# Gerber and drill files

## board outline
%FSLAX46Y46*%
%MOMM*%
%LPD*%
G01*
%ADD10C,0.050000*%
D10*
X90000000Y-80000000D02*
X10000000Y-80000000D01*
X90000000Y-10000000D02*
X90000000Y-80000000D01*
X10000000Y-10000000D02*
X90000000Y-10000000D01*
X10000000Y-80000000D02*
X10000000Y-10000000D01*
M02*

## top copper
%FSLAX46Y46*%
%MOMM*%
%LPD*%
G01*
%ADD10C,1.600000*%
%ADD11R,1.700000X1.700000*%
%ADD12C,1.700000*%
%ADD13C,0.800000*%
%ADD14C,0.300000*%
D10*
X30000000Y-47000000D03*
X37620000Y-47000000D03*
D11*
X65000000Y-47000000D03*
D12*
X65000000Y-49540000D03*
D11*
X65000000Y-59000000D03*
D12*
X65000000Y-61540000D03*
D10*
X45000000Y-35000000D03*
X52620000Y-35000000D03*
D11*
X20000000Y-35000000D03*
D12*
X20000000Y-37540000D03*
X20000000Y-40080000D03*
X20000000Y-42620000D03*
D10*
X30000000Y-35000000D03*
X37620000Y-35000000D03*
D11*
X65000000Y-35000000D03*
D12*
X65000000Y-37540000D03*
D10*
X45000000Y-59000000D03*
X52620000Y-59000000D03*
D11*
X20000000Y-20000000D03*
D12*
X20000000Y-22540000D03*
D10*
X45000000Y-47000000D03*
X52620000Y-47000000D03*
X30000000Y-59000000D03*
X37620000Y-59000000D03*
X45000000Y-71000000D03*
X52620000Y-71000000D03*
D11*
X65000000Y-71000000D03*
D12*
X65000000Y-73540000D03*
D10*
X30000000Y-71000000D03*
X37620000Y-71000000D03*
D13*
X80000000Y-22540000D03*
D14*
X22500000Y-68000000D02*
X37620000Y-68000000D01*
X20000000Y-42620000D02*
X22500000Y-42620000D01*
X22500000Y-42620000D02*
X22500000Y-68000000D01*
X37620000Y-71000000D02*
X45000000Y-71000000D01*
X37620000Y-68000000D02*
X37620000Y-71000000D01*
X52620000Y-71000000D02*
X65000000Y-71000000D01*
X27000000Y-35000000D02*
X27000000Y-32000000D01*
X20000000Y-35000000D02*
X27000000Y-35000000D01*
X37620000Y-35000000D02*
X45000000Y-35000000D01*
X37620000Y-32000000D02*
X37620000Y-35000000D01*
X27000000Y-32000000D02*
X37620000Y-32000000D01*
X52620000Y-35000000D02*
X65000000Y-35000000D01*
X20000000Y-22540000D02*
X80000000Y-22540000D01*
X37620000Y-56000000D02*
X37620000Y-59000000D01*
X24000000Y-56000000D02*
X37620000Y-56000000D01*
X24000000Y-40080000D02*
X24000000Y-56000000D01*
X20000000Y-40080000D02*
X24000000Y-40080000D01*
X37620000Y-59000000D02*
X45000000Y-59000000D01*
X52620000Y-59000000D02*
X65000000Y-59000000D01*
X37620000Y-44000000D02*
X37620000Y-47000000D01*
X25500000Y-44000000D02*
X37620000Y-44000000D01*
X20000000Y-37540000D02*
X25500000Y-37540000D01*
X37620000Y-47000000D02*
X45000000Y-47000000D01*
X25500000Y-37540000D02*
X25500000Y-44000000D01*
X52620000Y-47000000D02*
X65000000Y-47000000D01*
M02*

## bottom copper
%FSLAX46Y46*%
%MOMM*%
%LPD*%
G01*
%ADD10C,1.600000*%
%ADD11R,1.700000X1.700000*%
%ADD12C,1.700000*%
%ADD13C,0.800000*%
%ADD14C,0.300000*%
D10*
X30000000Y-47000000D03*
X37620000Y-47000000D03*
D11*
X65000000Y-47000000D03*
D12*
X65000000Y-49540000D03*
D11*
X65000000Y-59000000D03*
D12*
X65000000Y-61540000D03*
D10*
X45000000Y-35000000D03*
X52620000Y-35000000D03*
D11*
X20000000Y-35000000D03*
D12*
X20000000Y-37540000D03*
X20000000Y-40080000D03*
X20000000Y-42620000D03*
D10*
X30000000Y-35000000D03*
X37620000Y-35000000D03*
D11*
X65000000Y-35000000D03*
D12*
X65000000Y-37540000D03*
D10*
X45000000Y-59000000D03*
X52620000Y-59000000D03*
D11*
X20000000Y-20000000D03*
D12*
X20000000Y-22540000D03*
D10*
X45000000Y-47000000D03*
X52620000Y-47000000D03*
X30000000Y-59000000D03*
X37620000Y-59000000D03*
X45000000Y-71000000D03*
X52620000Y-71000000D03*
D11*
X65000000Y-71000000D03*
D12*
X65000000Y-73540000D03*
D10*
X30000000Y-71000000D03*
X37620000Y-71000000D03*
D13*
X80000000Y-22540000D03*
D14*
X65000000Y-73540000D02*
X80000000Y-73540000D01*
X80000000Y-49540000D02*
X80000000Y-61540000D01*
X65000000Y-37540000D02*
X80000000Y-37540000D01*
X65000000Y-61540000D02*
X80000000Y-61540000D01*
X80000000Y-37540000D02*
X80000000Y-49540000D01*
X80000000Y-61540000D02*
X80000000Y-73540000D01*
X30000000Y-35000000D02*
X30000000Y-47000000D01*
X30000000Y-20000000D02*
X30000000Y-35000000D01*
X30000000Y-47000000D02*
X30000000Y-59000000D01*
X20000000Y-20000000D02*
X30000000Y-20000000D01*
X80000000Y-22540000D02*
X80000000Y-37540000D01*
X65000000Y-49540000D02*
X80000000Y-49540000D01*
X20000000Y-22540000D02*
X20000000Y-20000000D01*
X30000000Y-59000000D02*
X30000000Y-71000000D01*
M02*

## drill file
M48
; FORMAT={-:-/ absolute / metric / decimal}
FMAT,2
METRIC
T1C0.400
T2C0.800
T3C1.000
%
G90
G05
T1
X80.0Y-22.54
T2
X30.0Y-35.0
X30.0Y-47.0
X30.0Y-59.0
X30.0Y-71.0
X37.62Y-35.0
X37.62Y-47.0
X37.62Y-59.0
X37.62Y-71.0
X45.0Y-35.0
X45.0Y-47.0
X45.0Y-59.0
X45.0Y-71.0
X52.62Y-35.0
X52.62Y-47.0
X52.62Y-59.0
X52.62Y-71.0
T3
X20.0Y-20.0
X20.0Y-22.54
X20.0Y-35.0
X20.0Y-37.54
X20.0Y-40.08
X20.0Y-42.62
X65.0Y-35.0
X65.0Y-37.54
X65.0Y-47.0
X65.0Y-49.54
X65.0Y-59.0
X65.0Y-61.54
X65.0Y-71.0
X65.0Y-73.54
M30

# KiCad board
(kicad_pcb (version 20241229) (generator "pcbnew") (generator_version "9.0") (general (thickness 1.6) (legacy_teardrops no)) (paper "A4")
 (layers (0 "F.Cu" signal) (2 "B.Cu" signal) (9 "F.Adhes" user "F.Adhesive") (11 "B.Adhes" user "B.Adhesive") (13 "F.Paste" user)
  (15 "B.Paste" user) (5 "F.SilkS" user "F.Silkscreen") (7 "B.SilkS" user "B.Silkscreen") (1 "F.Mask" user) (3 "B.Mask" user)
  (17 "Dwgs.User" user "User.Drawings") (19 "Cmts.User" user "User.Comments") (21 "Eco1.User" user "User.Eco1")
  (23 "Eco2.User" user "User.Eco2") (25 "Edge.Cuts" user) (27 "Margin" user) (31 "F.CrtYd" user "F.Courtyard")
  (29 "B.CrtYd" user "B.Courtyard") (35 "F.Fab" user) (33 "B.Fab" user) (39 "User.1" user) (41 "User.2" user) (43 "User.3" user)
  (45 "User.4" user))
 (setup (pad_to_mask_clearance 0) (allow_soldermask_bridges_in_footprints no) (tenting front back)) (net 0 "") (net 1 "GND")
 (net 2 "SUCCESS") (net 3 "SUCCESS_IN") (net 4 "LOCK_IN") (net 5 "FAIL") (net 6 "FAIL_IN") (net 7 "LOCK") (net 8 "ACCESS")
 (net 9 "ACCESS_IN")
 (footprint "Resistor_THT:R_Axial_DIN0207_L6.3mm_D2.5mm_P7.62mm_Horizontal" (layer "F.Cu") (at 30 47)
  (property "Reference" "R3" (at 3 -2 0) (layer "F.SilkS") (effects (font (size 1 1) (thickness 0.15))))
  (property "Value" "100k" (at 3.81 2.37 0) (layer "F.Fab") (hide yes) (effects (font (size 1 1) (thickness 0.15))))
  (pad "1" thru_hole circle (at 0 0) (size 1.6 1.6) (drill 0.8) (layers "*.Cu" "*.Mask") (remove_unused_layers no) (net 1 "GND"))
  (pad "2" thru_hole circle (at 7.62 0) (size 1.6 1.6) (drill 0.8) (layers "*.Cu" "*.Mask") (remove_unused_layers no) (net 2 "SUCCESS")))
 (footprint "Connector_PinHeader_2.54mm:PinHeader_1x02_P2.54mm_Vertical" (layer "F.Cu") (at 65 47)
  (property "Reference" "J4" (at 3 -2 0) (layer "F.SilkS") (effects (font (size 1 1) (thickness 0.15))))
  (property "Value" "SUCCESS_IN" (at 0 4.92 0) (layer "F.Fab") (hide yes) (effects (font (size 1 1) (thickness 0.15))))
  (pad "1" thru_hole rect (at 0 0) (size 1.7 1.7) (drill 1) (layers "*.Cu" "*.Mask") (remove_unused_layers no) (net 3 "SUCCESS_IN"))
  (pad "2" thru_hole circle (at 0 2.54) (size 1.7 1.7) (drill 1) (layers "*.Cu" "*.Mask") (remove_unused_layers no) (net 1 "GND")))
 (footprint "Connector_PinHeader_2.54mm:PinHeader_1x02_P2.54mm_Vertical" (layer "F.Cu") (at 65 59)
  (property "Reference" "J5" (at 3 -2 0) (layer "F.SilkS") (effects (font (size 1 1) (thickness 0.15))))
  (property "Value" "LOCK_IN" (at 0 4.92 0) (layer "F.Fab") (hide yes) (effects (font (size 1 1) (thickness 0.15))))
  (pad "1" thru_hole rect (at 0 0) (size 1.7 1.7) (drill 1) (layers "*.Cu" "*.Mask") (remove_unused_layers no) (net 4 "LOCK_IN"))
  (pad "2" thru_hole circle (at 0 2.54) (size 1.7 1.7) (drill 1) (layers "*.Cu" "*.Mask") (remove_unused_layers no) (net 1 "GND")))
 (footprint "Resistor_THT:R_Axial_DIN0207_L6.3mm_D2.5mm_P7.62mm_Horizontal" (layer "F.Cu") (at 45 35)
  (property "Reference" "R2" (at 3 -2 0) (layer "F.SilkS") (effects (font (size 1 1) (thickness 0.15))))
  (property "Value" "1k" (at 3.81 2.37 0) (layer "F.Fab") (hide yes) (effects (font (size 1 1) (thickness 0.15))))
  (pad "1" thru_hole circle (at 0 0) (size 1.6 1.6) (drill 0.8) (layers "*.Cu" "*.Mask") (remove_unused_layers no) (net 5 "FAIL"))
  (pad "2" thru_hole circle (at 7.62 0) (size 1.6 1.6) (drill 0.8) (layers "*.Cu" "*.Mask") (remove_unused_layers no) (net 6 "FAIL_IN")))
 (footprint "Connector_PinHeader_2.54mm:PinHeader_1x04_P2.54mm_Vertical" (layer "F.Cu") (at 20 35)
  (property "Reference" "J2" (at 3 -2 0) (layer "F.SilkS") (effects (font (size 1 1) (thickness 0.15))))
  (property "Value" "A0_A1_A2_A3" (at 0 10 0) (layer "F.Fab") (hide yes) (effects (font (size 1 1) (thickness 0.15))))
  (pad "1" thru_hole rect (at 0 0) (size 1.7 1.7) (drill 1) (layers "*.Cu" "*.Mask") (remove_unused_layers no) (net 5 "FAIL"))
  (pad "2" thru_hole circle (at 0 2.54) (size 1.7 1.7) (drill 1) (layers "*.Cu" "*.Mask") (remove_unused_layers no) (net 2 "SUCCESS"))
  (pad "3" thru_hole circle (at 0 5.08) (size 1.7 1.7) (drill 1) (layers "*.Cu" "*.Mask") (remove_unused_layers no) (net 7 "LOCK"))
  (pad "4" thru_hole circle (at 0 7.62) (size 1.7 1.7) (drill 1) (layers "*.Cu" "*.Mask") (remove_unused_layers no) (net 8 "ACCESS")))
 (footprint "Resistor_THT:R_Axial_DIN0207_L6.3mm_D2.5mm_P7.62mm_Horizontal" (layer "F.Cu") (at 30 35)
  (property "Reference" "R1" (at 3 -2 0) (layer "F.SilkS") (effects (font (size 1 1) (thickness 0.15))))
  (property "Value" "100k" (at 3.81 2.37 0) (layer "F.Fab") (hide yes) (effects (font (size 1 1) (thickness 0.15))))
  (pad "1" thru_hole circle (at 0 0) (size 1.6 1.6) (drill 0.8) (layers "*.Cu" "*.Mask") (remove_unused_layers no) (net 1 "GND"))
  (pad "2" thru_hole circle (at 7.62 0) (size 1.6 1.6) (drill 0.8) (layers "*.Cu" "*.Mask") (remove_unused_layers no) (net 5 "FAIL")))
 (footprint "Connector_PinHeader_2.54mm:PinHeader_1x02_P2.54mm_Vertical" (layer "F.Cu") (at 65 35)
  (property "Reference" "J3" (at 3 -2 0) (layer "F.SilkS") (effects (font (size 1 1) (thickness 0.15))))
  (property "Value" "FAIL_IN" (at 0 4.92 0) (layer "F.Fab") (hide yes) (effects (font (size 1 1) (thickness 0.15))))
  (pad "1" thru_hole rect (at 0 0) (size 1.7 1.7) (drill 1) (layers "*.Cu" "*.Mask") (remove_unused_layers no) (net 6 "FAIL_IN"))
  (pad "2" thru_hole circle (at 0 2.54) (size 1.7 1.7) (drill 1) (layers "*.Cu" "*.Mask") (remove_unused_layers no) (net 1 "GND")))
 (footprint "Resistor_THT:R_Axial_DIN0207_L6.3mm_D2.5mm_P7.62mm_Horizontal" (layer "F.Cu") (at 45 59)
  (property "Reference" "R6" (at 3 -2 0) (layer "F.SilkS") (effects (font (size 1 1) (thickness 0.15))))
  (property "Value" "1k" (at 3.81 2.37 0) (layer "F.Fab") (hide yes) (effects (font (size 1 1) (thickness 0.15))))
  (pad "1" thru_hole circle (at 0 0) (size 1.6 1.6) (drill 0.8) (layers "*.Cu" "*.Mask") (remove_unused_layers no) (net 7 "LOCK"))
  (pad "2" thru_hole circle (at 7.62 0) (size 1.6 1.6) (drill 0.8) (layers "*.Cu" "*.Mask") (remove_unused_layers no) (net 4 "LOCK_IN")))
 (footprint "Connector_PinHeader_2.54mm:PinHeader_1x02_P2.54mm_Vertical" (layer "F.Cu") (at 20 20)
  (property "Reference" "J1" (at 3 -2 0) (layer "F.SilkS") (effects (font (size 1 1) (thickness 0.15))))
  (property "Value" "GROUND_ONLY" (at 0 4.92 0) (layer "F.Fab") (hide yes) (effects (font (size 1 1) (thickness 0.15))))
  (pad "1" thru_hole rect (at 0 0) (size 1.7 1.7) (drill 1) (layers "*.Cu" "*.Mask") (remove_unused_layers no) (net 1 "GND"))
  (pad "2" thru_hole circle (at 0 2.54) (size 1.7 1.7) (drill 1) (layers "*.Cu" "*.Mask") (remove_unused_layers no) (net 1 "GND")))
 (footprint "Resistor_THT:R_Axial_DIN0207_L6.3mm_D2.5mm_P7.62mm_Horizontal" (layer "F.Cu") (at 45 47)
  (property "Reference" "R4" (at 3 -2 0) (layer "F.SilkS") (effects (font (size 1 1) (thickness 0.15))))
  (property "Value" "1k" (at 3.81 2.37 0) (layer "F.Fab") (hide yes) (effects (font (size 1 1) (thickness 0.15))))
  (pad "1" thru_hole circle (at 0 0) (size 1.6 1.6) (drill 0.8) (layers "*.Cu" "*.Mask") (remove_unused_layers no) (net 2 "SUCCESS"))
  (pad "2" thru_hole circle (at 7.62 0) (size 1.6 1.6) (drill 0.8) (layers "*.Cu" "*.Mask") (remove_unused_layers no) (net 3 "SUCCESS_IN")))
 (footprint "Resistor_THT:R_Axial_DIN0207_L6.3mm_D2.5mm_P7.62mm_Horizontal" (layer "F.Cu") (at 30 59)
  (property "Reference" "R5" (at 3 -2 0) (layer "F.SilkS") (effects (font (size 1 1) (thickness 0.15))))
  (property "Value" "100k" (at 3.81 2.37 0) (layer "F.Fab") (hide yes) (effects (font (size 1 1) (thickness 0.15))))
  (pad "1" thru_hole circle (at 0 0) (size 1.6 1.6) (drill 0.8) (layers "*.Cu" "*.Mask") (remove_unused_layers no) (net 1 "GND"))
  (pad "2" thru_hole circle (at 7.62 0) (size 1.6 1.6) (drill 0.8) (layers "*.Cu" "*.Mask") (remove_unused_layers no) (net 7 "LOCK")))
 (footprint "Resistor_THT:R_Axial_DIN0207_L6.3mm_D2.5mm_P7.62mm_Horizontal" (layer "F.Cu") (at 45 71)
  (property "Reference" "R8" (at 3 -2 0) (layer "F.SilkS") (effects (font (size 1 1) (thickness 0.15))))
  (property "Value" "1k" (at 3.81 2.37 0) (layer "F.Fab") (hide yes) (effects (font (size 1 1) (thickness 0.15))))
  (pad "1" thru_hole circle (at 0 0) (size 1.6 1.6) (drill 0.8) (layers "*.Cu" "*.Mask") (remove_unused_layers no) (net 8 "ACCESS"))
  (pad "2" thru_hole circle (at 7.62 0) (size 1.6 1.6) (drill 0.8) (layers "*.Cu" "*.Mask") (remove_unused_layers no) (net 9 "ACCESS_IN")))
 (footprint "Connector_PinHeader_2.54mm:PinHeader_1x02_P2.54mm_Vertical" (layer "F.Cu") (at 65 71)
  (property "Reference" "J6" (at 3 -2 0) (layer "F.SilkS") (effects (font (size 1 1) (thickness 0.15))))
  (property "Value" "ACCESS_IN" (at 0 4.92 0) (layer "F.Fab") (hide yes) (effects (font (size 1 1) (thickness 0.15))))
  (pad "1" thru_hole rect (at 0 0) (size 1.7 1.7) (drill 1) (layers "*.Cu" "*.Mask") (remove_unused_layers no) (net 9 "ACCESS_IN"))
  (pad "2" thru_hole circle (at 0 2.54) (size 1.7 1.7) (drill 1) (layers "*.Cu" "*.Mask") (remove_unused_layers no) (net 1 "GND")))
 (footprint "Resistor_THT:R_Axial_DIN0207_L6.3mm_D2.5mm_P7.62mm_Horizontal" (layer "F.Cu") (at 30 71)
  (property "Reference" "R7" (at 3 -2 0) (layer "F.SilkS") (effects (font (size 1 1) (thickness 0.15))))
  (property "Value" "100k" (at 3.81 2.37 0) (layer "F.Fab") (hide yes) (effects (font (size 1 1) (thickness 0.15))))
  (pad "1" thru_hole circle (at 0 0) (size 1.6 1.6) (drill 0.8) (layers "*.Cu" "*.Mask") (remove_unused_layers no) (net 1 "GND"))
  (pad "2" thru_hole circle (at 7.62 0) (size 1.6 1.6) (drill 0.8) (layers "*.Cu" "*.Mask") (remove_unused_layers no) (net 8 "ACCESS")))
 (gr_line (start 90 80) (end 10 80) (stroke (width 0.05) (type default)) (layer "Edge.Cuts"))
 (gr_line (start 90 10) (end 90 80) (stroke (width 0.05) (type default)) (layer "Edge.Cuts"))
 (gr_line (start 10 10) (end 90 10) (stroke (width 0.05) (type default)) (layer "Edge.Cuts"))
 (gr_line (start 10 80) (end 10 10) (stroke (width 0.05) (type default)) (layer "Edge.Cuts"))
 (segment (start 22.5 68) (end 37.62 68) (width 0.3) (layer "F.Cu") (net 8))
 (segment (start 20 42.62) (end 22.5 42.62) (width 0.3) (layer "F.Cu") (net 8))
 (segment (start 22.5 42.62) (end 22.5 68) (width 0.3) (layer "F.Cu") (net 8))
 (segment (start 37.62 71) (end 45 71) (width 0.3) (layer "F.Cu") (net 8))
 (segment (start 37.62 68) (end 37.62 71) (width 0.3) (layer "F.Cu") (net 8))
 (segment (start 52.62 71) (end 65 71) (width 0.3) (layer "F.Cu") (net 9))
 (segment (start 27 35) (end 27 32) (width 0.3) (layer "F.Cu") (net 5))
 (segment (start 20 35) (end 27 35) (width 0.3) (layer "F.Cu") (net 5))
 (segment (start 37.62 35) (end 45 35) (width 0.3) (layer "F.Cu") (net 5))
 (segment (start 37.62 32) (end 37.62 35) (width 0.3) (layer "F.Cu") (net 5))
 (segment (start 27 32) (end 37.62 32) (width 0.3) (layer "F.Cu") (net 5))
 (segment (start 52.62 35) (end 65 35) (width 0.3) (layer "F.Cu") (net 6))
 (segment (start 20 22.54) (end 80 22.54) (width 0.3) (layer "F.Cu") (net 1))
 (via (at 80 22.54) (size 0.8) (drill 0.4) (layers "F.Cu" "B.Cu") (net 1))
 (segment (start 65 73.54) (end 80 73.54) (width 0.3) (layer "B.Cu") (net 1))
 (segment (start 80 49.54) (end 80 61.54) (width 0.3) (layer "B.Cu") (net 1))
 (segment (start 65 37.54) (end 80 37.54) (width 0.3) (layer "B.Cu") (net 1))
 (segment (start 65 61.54) (end 80 61.54) (width 0.3) (layer "B.Cu") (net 1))
 (segment (start 80 37.54) (end 80 49.54) (width 0.3) (layer "B.Cu") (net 1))
 (segment (start 80 61.54) (end 80 73.54) (width 0.3) (layer "B.Cu") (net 1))
 (segment (start 30 35) (end 30 47) (width 0.3) (layer "B.Cu") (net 1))
 (segment (start 30 20) (end 30 35) (width 0.3) (layer "B.Cu") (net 1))
 (segment (start 30 47) (end 30 59) (width 0.3) (layer "B.Cu") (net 1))
 (segment (start 20 20) (end 30 20) (width 0.3) (layer "B.Cu") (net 1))
 (segment (start 80 22.54) (end 80 37.54) (width 0.3) (layer "B.Cu") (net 1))
 (segment (start 65 49.54) (end 80 49.54) (width 0.3) (layer "B.Cu") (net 1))
 (segment (start 20 22.54) (end 20 20) (width 0.3) (layer "B.Cu") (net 1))
 (segment (start 30 59) (end 30 71) (width 0.3) (layer "B.Cu") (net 1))
 (segment (start 37.62 56) (end 37.62 59) (width 0.3) (layer "F.Cu") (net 7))
 (segment (start 24 56) (end 37.62 56) (width 0.3) (layer "F.Cu") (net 7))
 (segment (start 24 40.08) (end 24 56) (width 0.3) (layer "F.Cu") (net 7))
 (segment (start 20 40.08) (end 24 40.08) (width 0.3) (layer "F.Cu") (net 7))
 (segment (start 37.62 59) (end 45 59) (width 0.3) (layer "F.Cu") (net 7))
 (segment (start 52.62 59) (end 65 59) (width 0.3) (layer "F.Cu") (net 4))
 (segment (start 37.62 44) (end 37.62 47) (width 0.3) (layer "F.Cu") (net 2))
 (segment (start 25.5 44) (end 37.62 44) (width 0.3) (layer "F.Cu") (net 2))
 (segment (start 20 37.54) (end 25.5 37.54) (width 0.3) (layer "F.Cu") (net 2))
 (segment (start 37.62 47) (end 45 47) (width 0.3) (layer "F.Cu") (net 2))
 (segment (start 25.5 37.54) (end 25.5 44) (width 0.3) (layer "F.Cu") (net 2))
 (segment (start 52.62 47) (end 65 47) (width 0.3) (layer "F.Cu") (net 3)))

